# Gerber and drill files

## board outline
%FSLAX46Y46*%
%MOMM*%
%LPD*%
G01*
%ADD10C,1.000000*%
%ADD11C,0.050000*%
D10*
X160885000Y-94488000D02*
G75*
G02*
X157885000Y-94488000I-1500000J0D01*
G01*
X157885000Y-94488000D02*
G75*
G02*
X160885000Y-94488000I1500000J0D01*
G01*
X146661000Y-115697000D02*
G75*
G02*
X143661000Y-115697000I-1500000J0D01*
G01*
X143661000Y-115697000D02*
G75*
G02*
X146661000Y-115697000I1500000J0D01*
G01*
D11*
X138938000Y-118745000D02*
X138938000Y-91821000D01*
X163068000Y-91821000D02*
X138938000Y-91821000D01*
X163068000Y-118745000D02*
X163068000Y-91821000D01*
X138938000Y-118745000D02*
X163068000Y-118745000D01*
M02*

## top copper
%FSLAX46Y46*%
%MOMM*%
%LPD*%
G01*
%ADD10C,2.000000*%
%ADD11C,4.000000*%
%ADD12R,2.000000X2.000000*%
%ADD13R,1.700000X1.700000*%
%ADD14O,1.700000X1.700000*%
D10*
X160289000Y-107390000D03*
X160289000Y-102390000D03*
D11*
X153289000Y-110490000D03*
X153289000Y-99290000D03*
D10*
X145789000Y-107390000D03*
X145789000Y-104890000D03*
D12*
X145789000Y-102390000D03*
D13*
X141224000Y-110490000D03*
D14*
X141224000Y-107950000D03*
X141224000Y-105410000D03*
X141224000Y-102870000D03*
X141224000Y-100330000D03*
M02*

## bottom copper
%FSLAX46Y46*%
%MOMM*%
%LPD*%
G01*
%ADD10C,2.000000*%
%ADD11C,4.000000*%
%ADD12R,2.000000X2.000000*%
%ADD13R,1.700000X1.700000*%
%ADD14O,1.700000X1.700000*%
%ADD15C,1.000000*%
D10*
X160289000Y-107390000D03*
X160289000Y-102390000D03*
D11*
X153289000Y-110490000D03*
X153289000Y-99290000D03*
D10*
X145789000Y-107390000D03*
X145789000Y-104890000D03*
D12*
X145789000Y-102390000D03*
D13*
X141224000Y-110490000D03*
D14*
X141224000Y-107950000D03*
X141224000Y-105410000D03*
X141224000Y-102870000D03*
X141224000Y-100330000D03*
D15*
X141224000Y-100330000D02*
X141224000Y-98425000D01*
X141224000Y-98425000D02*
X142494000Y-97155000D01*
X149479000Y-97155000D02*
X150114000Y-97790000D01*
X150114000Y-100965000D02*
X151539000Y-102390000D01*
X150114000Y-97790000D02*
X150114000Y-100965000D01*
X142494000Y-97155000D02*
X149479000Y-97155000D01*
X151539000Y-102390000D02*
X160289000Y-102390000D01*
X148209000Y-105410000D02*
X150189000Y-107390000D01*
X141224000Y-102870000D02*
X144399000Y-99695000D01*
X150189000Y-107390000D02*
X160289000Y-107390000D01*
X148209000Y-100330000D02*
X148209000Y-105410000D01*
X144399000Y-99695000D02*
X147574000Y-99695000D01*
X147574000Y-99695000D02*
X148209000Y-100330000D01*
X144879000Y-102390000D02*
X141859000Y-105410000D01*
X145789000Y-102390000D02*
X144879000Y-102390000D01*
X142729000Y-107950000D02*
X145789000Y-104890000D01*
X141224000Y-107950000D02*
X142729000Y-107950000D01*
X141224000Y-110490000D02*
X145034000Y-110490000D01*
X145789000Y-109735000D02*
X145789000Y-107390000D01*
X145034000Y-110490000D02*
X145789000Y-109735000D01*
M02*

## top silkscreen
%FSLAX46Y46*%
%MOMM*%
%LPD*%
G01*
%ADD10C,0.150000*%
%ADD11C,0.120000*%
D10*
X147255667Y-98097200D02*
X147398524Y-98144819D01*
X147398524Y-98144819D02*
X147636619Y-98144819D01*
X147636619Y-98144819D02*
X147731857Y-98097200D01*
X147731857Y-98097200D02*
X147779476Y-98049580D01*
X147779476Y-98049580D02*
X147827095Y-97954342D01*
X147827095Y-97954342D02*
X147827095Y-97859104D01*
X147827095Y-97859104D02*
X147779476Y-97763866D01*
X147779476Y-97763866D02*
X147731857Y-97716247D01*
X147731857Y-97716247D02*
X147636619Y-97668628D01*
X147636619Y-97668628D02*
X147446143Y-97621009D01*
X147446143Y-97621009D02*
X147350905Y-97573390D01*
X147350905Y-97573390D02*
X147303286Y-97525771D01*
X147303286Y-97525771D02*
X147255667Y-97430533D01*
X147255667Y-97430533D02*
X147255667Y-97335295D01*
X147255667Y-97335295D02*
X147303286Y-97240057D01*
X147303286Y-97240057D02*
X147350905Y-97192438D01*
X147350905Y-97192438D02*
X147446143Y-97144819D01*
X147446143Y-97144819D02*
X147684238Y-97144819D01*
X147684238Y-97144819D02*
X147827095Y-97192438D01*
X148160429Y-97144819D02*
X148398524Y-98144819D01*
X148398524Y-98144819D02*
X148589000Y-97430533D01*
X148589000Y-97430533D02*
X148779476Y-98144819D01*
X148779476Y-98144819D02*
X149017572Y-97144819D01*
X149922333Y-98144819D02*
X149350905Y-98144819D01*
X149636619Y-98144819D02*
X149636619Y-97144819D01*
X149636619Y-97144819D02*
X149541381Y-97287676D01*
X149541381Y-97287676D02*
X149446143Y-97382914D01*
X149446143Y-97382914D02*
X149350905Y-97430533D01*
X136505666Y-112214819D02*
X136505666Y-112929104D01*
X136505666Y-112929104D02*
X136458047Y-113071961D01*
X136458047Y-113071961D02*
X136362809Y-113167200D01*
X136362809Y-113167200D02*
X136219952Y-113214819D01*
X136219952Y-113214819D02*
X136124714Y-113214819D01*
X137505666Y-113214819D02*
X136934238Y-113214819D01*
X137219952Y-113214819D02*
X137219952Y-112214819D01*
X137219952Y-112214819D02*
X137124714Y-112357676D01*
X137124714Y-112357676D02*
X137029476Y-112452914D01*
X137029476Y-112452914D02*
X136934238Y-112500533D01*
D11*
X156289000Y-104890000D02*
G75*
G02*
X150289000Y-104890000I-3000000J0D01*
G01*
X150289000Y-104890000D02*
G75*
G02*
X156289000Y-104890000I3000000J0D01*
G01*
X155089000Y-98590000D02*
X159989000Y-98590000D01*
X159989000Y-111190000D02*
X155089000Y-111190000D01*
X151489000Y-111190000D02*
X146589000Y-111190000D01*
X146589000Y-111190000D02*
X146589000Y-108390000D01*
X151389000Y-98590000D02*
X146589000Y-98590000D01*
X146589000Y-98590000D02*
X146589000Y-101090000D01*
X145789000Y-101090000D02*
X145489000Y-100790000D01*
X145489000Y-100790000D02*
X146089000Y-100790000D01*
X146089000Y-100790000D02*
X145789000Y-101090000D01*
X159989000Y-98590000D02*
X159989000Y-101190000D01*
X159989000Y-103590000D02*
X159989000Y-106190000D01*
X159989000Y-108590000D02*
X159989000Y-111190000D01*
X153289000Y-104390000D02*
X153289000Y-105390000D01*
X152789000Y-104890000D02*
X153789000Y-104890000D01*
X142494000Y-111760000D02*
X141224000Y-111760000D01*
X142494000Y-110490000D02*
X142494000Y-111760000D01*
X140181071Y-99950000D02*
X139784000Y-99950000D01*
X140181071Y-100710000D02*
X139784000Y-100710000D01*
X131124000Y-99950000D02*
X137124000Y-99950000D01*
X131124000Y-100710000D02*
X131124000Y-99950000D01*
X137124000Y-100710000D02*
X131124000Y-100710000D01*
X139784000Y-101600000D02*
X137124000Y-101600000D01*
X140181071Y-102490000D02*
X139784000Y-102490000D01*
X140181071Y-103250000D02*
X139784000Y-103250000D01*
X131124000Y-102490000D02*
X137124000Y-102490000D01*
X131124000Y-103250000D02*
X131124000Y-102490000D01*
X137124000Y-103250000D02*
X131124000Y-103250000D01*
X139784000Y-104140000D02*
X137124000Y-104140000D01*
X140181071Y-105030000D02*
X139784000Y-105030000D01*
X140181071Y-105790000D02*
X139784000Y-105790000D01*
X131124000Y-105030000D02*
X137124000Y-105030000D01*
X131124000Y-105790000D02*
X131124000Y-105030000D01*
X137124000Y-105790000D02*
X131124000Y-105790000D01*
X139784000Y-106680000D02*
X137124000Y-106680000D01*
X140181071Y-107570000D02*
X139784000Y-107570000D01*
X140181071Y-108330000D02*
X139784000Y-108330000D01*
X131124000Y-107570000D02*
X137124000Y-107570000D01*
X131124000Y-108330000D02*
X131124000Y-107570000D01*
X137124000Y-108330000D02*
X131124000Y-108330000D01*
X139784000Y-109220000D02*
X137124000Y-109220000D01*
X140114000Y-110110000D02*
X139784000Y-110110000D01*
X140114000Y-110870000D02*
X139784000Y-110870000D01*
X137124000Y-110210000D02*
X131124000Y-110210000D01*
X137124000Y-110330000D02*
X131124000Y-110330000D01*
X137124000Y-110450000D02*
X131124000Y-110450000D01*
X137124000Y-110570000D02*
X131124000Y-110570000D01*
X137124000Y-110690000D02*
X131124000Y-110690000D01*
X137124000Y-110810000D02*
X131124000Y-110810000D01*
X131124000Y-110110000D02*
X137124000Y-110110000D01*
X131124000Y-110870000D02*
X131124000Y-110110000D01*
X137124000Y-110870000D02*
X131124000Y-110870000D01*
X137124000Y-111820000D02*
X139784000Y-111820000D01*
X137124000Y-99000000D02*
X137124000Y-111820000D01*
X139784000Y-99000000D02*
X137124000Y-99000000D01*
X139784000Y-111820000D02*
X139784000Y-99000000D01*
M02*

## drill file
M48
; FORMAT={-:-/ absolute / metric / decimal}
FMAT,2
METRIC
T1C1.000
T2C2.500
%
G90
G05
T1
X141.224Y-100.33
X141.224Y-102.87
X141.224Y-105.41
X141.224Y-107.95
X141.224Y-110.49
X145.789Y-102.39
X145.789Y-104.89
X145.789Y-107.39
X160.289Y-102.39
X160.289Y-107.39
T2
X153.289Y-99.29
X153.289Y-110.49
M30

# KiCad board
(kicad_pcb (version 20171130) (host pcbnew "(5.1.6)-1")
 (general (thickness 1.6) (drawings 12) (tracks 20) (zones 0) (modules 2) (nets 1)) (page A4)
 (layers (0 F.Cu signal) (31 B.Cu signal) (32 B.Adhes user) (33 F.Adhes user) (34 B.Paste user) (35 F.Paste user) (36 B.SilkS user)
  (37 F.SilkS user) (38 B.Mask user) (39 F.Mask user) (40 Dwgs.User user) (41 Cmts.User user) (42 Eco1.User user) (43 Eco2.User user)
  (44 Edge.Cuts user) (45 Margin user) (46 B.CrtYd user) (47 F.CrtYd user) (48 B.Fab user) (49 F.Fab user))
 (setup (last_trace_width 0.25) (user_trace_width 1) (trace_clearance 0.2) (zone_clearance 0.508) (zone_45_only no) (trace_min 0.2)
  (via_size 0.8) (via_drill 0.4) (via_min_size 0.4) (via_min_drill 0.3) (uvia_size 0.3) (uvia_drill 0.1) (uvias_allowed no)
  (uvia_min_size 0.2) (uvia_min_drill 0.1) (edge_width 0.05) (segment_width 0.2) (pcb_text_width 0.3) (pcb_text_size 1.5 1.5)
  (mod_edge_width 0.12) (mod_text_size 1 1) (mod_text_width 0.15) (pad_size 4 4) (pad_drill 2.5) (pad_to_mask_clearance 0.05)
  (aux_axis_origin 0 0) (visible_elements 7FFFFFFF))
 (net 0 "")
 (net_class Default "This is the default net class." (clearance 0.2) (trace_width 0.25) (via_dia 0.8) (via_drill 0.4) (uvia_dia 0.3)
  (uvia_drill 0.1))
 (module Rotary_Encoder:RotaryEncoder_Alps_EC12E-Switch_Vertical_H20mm (layer F.Cu) (at 145.789 102.39)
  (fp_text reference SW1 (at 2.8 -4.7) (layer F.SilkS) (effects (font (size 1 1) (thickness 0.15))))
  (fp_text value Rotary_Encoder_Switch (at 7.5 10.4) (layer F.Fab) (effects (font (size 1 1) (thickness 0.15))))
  (fp_circle (center 7.5 2.5) (end 10.5 2.5) (layer F.SilkS) (width 0.12))
  (fp_line (start 9.3 -3.8) (end 14.2 -3.8) (layer F.SilkS) (width 0.12))
  (fp_line (start 14.2 8.8) (end 9.3 8.8) (layer F.SilkS) (width 0.12))
  (fp_line (start 5.7 8.8) (end 0.8 8.8) (layer F.SilkS) (width 0.12))
  (fp_line (start 0.8 8.8) (end 0.8 6) (layer F.SilkS) (width 0.12))
  (fp_line (start 5.6 -3.8) (end 0.8 -3.8) (layer F.SilkS) (width 0.12))
  (fp_line (start 0.8 -3.8) (end 0.8 -1.3) (layer F.SilkS) (width 0.12))
  (fp_line (start 0 -1.3) (end -0.3 -1.6) (layer F.SilkS) (width 0.12))
  (fp_line (start -0.3 -1.6) (end 0.3 -1.6) (layer F.SilkS) (width 0.12))
  (fp_line (start 0.3 -1.6) (end 0 -1.3) (layer F.SilkS) (width 0.12))
  (fp_line (start 14.2 -3.8) (end 14.2 -1.2) (layer F.SilkS) (width 0.12))
  (fp_line (start 14.2 1.2) (end 14.2 3.8) (layer F.SilkS) (width 0.12))
  (fp_line (start 14.2 6.2) (end 14.2 8.8) (layer F.SilkS) (width 0.12))
  (fp_line (start 7.5 2) (end 7.5 3) (layer F.SilkS) (width 0.12))
  (fp_line (start 7 2.5) (end 8 2.5) (layer F.SilkS) (width 0.12))
  (pad S2 thru_hole circle (at 14.5 5) (size 2 2) (drill 1) (layers *.Cu *.Mask))
  (pad S1 thru_hole circle (at 14.5 0) (size 2 2) (drill 1) (layers *.Cu *.Mask))
  (pad MP thru_hole circle (at 7.5 8.1) (size 4 4) (drill 2.5) (layers *.Cu *.Mask))
  (pad MP thru_hole circle (at 7.5 -3.1) (size 4 4) (drill 2.5) (layers *.Cu *.Mask))
  (pad B thru_hole circle (at 0 5) (size 2 2) (drill 1) (layers *.Cu *.Mask))
  (pad C thru_hole circle (at 0 2.5) (size 2 2) (drill 1) (layers *.Cu *.Mask))
  (pad A thru_hole rect (at 0 0) (size 2 2) (drill 1) (layers *.Cu *.Mask)))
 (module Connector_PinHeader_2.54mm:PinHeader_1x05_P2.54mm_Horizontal (layer F.Cu) (at 141.224 110.49 180)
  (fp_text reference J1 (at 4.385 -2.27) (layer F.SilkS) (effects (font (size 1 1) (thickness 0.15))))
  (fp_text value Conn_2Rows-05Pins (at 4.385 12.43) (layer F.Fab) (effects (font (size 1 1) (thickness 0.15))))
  (fp_line (start -1.27 -1.27) (end 0 -1.27) (layer F.SilkS) (width 0.12))
  (fp_line (start -1.27 0) (end -1.27 -1.27) (layer F.SilkS) (width 0.12))
  (fp_line (start 1.042929 10.54) (end 1.44 10.54) (layer F.SilkS) (width 0.12))
  (fp_line (start 1.042929 9.78) (end 1.44 9.78) (layer F.SilkS) (width 0.12))
  (fp_line (start 10.1 10.54) (end 4.1 10.54) (layer F.SilkS) (width 0.12))
  (fp_line (start 10.1 9.78) (end 10.1 10.54) (layer F.SilkS) (width 0.12))
  (fp_line (start 4.1 9.78) (end 10.1 9.78) (layer F.SilkS) (width 0.12))
  (fp_line (start 1.44 8.89) (end 4.1 8.89) (layer F.SilkS) (width 0.12))
  (fp_line (start 1.042929 8) (end 1.44 8) (layer F.SilkS) (width 0.12))
  (fp_line (start 1.042929 7.24) (end 1.44 7.24) (layer F.SilkS) (width 0.12))
  (fp_line (start 10.1 8) (end 4.1 8) (layer F.SilkS) (width 0.12))
  (fp_line (start 10.1 7.24) (end 10.1 8) (layer F.SilkS) (width 0.12))
  (fp_line (start 4.1 7.24) (end 10.1 7.24) (layer F.SilkS) (width 0.12))
  (fp_line (start 1.44 6.35) (end 4.1 6.35) (layer F.SilkS) (width 0.12))
  (fp_line (start 1.042929 5.46) (end 1.44 5.46) (layer F.SilkS) (width 0.12))
  (fp_line (start 1.042929 4.7) (end 1.44 4.7) (layer F.SilkS) (width 0.12))
  (fp_line (start 10.1 5.46) (end 4.1 5.46) (layer F.SilkS) (width 0.12))
  (fp_line (start 10.1 4.7) (end 10.1 5.46) (layer F.SilkS) (width 0.12))
  (fp_line (start 4.1 4.7) (end 10.1 4.7) (layer F.SilkS) (width 0.12))
  (fp_line (start 1.44 3.81) (end 4.1 3.81) (layer F.SilkS) (width 0.12))
  (fp_line (start 1.042929 2.92) (end 1.44 2.92) (layer F.SilkS) (width 0.12))
  (fp_line (start 1.042929 2.16) (end 1.44 2.16) (layer F.SilkS) (width 0.12))
  (fp_line (start 10.1 2.92) (end 4.1 2.92) (layer F.SilkS) (width 0.12))
  (fp_line (start 10.1 2.16) (end 10.1 2.92) (layer F.SilkS) (width 0.12))
  (fp_line (start 4.1 2.16) (end 10.1 2.16) (layer F.SilkS) (width 0.12))
  (fp_line (start 1.44 1.27) (end 4.1 1.27) (layer F.SilkS) (width 0.12))
  (fp_line (start 1.11 0.38) (end 1.44 0.38) (layer F.SilkS) (width 0.12))
  (fp_line (start 1.11 -0.38) (end 1.44 -0.38) (layer F.SilkS) (width 0.12))
  (fp_line (start 4.1 0.28) (end 10.1 0.28) (layer F.SilkS) (width 0.12))
  (fp_line (start 4.1 0.16) (end 10.1 0.16) (layer F.SilkS) (width 0.12))
  (fp_line (start 4.1 0.04) (end 10.1 0.04) (layer F.SilkS) (width 0.12))
  (fp_line (start 4.1 -0.08) (end 10.1 -0.08) (layer F.SilkS) (width 0.12))
  (fp_line (start 4.1 -0.2) (end 10.1 -0.2) (layer F.SilkS) (width 0.12))
  (fp_line (start 4.1 -0.32) (end 10.1 -0.32) (layer F.SilkS) (width 0.12))
  (fp_line (start 10.1 0.38) (end 4.1 0.38) (layer F.SilkS) (width 0.12))
  (fp_line (start 10.1 -0.38) (end 10.1 0.38) (layer F.SilkS) (width 0.12))
  (fp_line (start 4.1 -0.38) (end 10.1 -0.38) (layer F.SilkS) (width 0.12))
  (fp_line (start 4.1 -1.33) (end 1.44 -1.33) (layer F.SilkS) (width 0.12))
  (fp_line (start 4.1 11.49) (end 4.1 -1.33) (layer F.SilkS) (width 0.12))
  (fp_line (start 1.44 11.49) (end 4.1 11.49) (layer F.SilkS) (width 0.12))
  (fp_line (start 1.44 -1.33) (end 1.44 11.49) (layer F.SilkS) (width 0.12))
  (pad 1 thru_hole rect (at 0 0 180) (size 1.7 1.7) (drill 1) (layers *.Cu *.Mask))
  (pad 2 thru_hole oval (at 0 2.54 180) (size 1.7 1.7) (drill 1) (layers *.Cu *.Mask))
  (pad 3 thru_hole oval (at 0 5.08 180) (size 1.7 1.7) (drill 1) (layers *.Cu *.Mask))
  (pad 4 thru_hole oval (at 0 7.62 180) (size 1.7 1.7) (drill 1) (layers *.Cu *.Mask))
  (pad 5 thru_hole oval (at 0 10.16 180) (size 1.7 1.7) (drill 1) (layers *.Cu *.Mask)))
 (gr_circle (center 159.385 94.488) (end 160.885 94.488) (layer Edge.Cuts) (width 1))
 (gr_circle (center 145.161 115.697) (end 146.661 115.697) (layer Edge.Cuts) (width 1))
 (gr_line (start 138.938 118.745) (end 138.938 91.821) (layer Edge.Cuts) (width 0.05))
 (gr_line (start 163.068 91.821) (end 138.938 91.821) (layer Edge.Cuts) (width 0.05))
 (gr_line (start 163.068 118.745) (end 163.068 91.821) (layer Edge.Cuts) (width 0.05))
 (gr_line (start 138.938 118.745) (end 163.068 118.745) (layer Edge.Cuts) (width 0.05))
 (segment (start 141.224 100.33) (end 141.224 98.425) (width 1) (layer B.Cu) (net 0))
 (segment (start 141.224 98.425) (end 142.494 97.155) (width 1) (layer B.Cu) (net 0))
 (segment (start 149.479 97.155) (end 150.114 97.79) (width 1) (layer B.Cu) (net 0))
 (segment (start 150.114 100.965) (end 151.539 102.39) (width 1) (layer B.Cu) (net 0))
 (segment (start 150.114 97.79) (end 150.114 100.965) (width 1) (layer B.Cu) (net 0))
 (segment (start 142.494 97.155) (end 149.479 97.155) (width 1) (layer B.Cu) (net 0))
 (segment (start 151.539 102.39) (end 160.289 102.39) (width 1) (layer B.Cu) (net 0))
 (segment (start 148.209 105.41) (end 150.189 107.39) (width 1) (layer B.Cu) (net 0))
 (segment (start 141.224 102.87) (end 144.399 99.695) (width 1) (layer B.Cu) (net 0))
 (segment (start 150.189 107.39) (end 160.289 107.39) (width 1) (layer B.Cu) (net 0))
 (segment (start 148.209 100.33) (end 148.209 105.41) (width 1) (layer B.Cu) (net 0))
 (segment (start 144.399 99.695) (end 147.574 99.695) (width 1) (layer B.Cu) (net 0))
 (segment (start 147.574 99.695) (end 148.209 100.33) (width 1) (layer B.Cu) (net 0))
 (segment (start 144.879 102.39) (end 141.859 105.41) (width 1) (layer B.Cu) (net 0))
 (segment (start 145.789 102.39) (end 144.879 102.39) (width 1) (layer B.Cu) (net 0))
 (segment (start 142.729 107.95) (end 145.789 104.89) (width 1) (layer B.Cu) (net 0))
 (segment (start 141.224 107.95) (end 142.729 107.95) (width 1) (layer B.Cu) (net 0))
 (segment (start 141.224 110.49) (end 145.034 110.49) (width 1) (layer B.Cu) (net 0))
 (segment (start 145.789 109.735) (end 145.789 107.39) (width 1) (layer B.Cu) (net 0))
 (segment (start 145.034 110.49) (end 145.789 109.735) (width 1) (layer B.Cu) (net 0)))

